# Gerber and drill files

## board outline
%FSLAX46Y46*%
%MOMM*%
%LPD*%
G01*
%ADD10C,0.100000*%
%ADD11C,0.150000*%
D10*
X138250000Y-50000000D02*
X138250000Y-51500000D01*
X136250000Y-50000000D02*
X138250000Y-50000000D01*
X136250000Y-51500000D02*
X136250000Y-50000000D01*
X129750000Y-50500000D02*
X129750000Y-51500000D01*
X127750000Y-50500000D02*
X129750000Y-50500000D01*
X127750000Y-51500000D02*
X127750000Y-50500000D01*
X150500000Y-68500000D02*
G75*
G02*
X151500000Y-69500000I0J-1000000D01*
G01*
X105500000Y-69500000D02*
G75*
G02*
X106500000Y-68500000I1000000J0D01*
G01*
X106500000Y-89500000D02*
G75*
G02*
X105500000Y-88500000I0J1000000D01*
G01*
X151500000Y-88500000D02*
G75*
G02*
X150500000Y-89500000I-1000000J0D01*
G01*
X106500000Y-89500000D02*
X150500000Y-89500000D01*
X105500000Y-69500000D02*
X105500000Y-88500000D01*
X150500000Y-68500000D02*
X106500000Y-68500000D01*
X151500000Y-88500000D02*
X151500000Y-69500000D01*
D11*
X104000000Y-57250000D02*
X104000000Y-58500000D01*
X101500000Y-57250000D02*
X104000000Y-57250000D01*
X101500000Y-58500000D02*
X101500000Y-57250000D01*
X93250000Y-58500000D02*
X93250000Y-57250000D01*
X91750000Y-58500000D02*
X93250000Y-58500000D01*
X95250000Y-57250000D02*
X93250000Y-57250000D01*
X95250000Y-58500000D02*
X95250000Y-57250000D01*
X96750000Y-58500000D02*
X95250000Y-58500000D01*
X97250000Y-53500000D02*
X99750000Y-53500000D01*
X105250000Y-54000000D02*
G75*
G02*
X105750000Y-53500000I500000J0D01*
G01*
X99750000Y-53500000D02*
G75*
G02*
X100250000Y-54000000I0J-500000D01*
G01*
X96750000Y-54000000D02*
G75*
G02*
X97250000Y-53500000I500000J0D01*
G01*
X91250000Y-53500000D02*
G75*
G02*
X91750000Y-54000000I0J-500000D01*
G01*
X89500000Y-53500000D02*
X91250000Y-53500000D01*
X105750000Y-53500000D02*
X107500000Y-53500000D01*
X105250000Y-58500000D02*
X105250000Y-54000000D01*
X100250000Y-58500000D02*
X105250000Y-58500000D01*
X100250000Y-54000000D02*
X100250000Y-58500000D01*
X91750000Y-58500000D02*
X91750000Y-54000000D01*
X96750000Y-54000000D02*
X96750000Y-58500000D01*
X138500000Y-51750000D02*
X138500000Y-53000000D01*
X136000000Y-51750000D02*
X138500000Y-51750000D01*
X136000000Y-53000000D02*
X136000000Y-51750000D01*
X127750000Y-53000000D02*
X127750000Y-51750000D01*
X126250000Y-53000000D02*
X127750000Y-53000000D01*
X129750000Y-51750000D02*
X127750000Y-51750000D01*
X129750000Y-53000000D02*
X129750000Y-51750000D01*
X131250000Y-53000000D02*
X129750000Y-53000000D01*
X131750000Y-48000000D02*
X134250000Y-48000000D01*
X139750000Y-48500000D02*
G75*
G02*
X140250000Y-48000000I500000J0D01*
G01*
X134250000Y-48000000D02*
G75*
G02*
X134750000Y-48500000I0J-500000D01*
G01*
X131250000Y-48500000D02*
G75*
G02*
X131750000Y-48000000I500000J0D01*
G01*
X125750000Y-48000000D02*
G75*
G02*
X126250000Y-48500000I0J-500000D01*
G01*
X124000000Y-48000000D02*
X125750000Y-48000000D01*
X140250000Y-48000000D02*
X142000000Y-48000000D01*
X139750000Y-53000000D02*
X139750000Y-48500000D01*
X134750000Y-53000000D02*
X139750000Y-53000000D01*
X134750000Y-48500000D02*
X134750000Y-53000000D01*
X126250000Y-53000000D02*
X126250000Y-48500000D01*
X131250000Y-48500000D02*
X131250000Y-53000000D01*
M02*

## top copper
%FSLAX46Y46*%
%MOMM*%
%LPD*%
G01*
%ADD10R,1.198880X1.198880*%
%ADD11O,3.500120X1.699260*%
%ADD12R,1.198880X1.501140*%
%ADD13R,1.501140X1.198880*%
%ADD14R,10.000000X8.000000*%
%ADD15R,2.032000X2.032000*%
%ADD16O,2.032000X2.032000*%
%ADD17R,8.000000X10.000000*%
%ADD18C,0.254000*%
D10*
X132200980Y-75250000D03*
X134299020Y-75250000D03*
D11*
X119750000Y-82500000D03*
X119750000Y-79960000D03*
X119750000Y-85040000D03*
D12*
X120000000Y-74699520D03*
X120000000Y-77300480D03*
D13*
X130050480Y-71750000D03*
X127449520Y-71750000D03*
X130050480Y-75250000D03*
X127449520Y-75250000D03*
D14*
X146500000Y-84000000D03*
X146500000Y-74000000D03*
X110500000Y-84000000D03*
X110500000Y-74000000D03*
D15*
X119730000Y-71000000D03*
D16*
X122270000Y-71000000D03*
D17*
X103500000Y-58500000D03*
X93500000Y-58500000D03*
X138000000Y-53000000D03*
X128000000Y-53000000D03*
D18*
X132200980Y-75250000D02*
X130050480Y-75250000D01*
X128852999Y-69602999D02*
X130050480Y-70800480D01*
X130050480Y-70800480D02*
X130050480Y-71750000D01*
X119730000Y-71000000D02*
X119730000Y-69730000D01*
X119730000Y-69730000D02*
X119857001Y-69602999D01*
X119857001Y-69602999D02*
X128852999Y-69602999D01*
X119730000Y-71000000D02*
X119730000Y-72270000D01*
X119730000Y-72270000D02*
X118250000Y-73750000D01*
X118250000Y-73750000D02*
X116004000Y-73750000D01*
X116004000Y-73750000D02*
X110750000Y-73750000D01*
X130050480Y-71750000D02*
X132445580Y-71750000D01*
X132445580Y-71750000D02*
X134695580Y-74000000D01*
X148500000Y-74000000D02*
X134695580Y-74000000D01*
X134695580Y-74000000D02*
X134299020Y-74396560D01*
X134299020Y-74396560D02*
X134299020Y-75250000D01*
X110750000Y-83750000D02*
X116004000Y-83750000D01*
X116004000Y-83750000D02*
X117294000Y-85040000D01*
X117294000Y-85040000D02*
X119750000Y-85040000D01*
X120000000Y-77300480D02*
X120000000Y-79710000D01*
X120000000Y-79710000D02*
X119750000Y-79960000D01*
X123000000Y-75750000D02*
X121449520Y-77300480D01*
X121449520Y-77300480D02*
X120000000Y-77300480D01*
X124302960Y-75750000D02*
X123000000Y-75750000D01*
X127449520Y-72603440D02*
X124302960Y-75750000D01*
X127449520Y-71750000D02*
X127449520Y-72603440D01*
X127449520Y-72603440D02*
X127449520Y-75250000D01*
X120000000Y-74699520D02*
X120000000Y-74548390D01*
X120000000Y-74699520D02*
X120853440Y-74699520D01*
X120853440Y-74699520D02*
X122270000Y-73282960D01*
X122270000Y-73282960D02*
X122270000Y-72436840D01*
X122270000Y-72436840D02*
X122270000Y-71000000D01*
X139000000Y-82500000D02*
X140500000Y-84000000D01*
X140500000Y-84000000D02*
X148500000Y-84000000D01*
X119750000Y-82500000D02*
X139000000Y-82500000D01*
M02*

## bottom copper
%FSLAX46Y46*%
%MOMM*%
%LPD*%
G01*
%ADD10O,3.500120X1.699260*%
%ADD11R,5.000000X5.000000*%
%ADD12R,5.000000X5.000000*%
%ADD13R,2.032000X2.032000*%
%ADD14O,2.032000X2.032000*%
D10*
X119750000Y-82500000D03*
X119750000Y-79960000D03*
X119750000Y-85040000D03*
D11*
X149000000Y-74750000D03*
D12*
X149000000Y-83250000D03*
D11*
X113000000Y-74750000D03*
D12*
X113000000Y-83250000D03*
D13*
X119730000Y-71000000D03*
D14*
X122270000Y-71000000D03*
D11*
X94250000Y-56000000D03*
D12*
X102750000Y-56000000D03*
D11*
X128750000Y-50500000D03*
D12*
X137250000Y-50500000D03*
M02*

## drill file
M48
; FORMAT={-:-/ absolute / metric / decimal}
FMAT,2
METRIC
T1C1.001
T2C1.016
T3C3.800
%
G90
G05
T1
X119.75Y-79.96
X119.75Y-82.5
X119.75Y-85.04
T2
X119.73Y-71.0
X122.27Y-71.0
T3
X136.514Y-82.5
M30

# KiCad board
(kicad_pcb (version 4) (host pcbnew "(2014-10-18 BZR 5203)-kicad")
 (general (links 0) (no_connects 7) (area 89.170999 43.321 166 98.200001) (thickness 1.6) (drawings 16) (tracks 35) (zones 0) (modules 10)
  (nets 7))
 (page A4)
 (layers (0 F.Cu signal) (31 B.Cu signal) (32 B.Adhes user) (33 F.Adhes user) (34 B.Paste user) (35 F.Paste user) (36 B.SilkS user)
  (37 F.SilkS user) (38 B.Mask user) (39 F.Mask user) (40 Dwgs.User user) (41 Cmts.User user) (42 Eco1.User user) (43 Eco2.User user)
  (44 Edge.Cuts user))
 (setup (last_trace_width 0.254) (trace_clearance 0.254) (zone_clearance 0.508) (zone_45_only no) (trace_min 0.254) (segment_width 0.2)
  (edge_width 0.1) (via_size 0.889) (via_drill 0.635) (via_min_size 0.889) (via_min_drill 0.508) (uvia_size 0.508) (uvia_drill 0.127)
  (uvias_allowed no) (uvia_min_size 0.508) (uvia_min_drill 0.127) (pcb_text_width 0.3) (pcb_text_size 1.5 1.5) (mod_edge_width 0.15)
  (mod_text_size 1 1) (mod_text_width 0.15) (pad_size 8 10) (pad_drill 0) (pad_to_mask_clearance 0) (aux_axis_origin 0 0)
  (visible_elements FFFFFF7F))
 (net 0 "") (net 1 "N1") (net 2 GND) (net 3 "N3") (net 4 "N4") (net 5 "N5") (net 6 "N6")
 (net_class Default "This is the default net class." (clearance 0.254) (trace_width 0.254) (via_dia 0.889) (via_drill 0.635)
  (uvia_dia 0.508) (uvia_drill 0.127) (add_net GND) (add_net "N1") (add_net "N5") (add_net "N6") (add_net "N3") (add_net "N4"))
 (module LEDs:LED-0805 (layer F.Cu) (at 133.25 75.25)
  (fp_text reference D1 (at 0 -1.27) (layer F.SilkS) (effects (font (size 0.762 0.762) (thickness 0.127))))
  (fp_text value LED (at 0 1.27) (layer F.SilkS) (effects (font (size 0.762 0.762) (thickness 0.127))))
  (pad 1 smd rect (at -1.04902 0) (size 1.19888 1.19888) (layers F.Cu F.Paste F.Mask) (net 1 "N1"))
  (pad 2 smd rect (at 1.04902 0) (size 1.19888 1.19888) (layers F.Cu F.Paste F.Mask) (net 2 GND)))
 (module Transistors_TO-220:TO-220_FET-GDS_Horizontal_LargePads (layer F.Cu) (at 119.75 82.5 270)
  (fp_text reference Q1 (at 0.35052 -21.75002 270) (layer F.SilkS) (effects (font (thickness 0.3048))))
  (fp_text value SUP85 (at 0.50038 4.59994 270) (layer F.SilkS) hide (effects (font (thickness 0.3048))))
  (pad D thru_hole oval (at 0 0) (size 3.50012 1.69926) (drill 1.00076) (layers *.Cu *.Mask F.SilkS) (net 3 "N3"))
  (pad G thru_hole oval (at -2.54 0) (size 3.50012 1.69926) (drill 1.00076) (layers *.Cu *.Mask F.SilkS) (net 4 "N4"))
  (pad S thru_hole oval (at 2.54 0) (size 3.50012 1.69926) (drill 1.00076) (layers *.Cu *.Mask F.SilkS) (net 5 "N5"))
  (pad "" np_thru_hole circle (at 0 -16.764) (size 3.79984 3.79984) (drill 3.79984) (layers *.Cu *.Mask F.SilkS)))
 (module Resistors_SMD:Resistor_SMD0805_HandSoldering (layer F.Cu) (at 120 76 270)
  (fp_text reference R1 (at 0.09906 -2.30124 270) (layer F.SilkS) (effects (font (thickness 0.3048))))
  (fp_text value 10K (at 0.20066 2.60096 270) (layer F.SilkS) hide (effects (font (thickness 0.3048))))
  (pad 1 smd rect (at -1.30048 0 270) (size 1.50114 1.19888) (layers F.Cu F.Paste F.Mask) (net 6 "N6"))
  (pad 2 smd rect (at 1.30048 0 270) (size 1.50114 1.19888) (layers F.Cu F.Paste F.Mask) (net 4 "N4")))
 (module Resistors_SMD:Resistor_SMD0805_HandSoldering (layer F.Cu) (at 128.75 71.75 180)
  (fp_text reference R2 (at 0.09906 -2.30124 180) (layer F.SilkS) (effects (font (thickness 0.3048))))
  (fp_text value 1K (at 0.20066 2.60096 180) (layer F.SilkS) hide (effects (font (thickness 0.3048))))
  (pad 1 smd rect (at -1.30048 0 180) (size 1.50114 1.19888) (layers F.Cu F.Paste F.Mask) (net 2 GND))
  (pad 2 smd rect (at 1.30048 0 180) (size 1.50114 1.19888) (layers F.Cu F.Paste F.Mask) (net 4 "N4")))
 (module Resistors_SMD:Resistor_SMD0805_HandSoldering (layer F.Cu) (at 128.75 75.25 180)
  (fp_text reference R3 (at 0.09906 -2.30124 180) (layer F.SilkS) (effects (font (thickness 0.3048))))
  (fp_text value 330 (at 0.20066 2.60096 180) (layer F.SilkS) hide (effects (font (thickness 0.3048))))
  (pad 1 smd rect (at -1.30048 0 180) (size 1.50114 1.19888) (layers F.Cu F.Paste F.Mask) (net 1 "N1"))
  (pad 2 smd rect (at 1.30048 0 180) (size 1.50114 1.19888) (layers F.Cu F.Paste F.Mask) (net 4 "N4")))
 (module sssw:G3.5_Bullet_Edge (layer F.Cu) (at 149 79 270)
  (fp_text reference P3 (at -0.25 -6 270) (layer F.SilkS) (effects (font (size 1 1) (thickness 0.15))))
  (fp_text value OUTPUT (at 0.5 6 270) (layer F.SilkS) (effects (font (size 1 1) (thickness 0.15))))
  (pad 1 smd rect (at -4.25 0 270) (size 5 5) (layers B.Cu F.Paste F.Mask) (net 2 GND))
  (pad 2 connect rect (at 4.25 0 270) (size 5 5) (layers B.Cu F.Mask) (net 3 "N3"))
  (pad 2 smd rect (at 5 2.5 270) (size 8 10) (layers F.Cu F.Paste F.Mask) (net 3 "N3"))
  (pad 1 smd rect (at -5 2.5 270) (size 8 10) (layers F.Cu F.Paste F.Mask) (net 2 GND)))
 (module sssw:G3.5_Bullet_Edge (layer F.Cu) (at 113 79 270)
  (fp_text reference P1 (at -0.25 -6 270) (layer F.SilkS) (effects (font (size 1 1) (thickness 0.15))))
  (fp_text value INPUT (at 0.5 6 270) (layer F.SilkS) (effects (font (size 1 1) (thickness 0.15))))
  (pad 1 smd rect (at -4.25 0 270) (size 5 5) (layers B.Cu F.Paste F.Mask) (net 2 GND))
  (pad 2 connect rect (at 4.25 0 270) (size 5 5) (layers B.Cu F.Mask) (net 5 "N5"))
  (pad 2 smd rect (at 5 2.5 270) (size 8 10) (layers F.Cu F.Paste F.Mask) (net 5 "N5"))
  (pad 1 smd rect (at -5 2.5 270) (size 8 10) (layers F.Cu F.Paste F.Mask) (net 2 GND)))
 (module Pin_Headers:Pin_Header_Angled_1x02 (layer F.Cu) (at 121 71)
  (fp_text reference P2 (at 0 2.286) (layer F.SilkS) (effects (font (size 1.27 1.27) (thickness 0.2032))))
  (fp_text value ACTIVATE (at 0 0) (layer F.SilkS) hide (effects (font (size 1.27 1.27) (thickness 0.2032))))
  (pad 1 thru_hole rect (at -1.27 0) (size 2.032 2.032) (drill 1.016) (layers *.Cu *.Mask F.SilkS) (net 2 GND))
  (pad 2 thru_hole oval (at 1.27 0) (size 2.032 2.032) (drill 1.016) (layers *.Cu *.Mask F.SilkS) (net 6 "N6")))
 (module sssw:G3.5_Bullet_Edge (layer F.Cu) (at 98.5 56)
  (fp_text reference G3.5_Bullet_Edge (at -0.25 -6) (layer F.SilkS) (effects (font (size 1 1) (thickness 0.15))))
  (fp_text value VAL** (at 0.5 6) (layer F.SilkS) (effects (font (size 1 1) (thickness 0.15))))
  (fp_line (start 5.5 1.25) (end 5.5 2.5) (layer Edge.Cuts) (width 0.15))
  (fp_line (start 3 1.25) (end 5.5 1.25) (layer Edge.Cuts) (width 0.15))
  (fp_line (start 3 2.5) (end 3 1.25) (layer Edge.Cuts) (width 0.15))
  (fp_line (start -5.25 2.5) (end -5.25 1.25) (layer Edge.Cuts) (width 0.15))
  (fp_line (start -6.75 2.5) (end -5.25 2.5) (layer Edge.Cuts) (width 0.15))
  (fp_line (start -3.25 1.25) (end -5.25 1.25) (layer Edge.Cuts) (width 0.15))
  (fp_line (start -3.25 2.5) (end -3.25 1.25) (layer Edge.Cuts) (width 0.15))
  (fp_line (start -1.75 2.5) (end -3.25 2.5) (layer Edge.Cuts) (width 0.15))
  (fp_line (start -1.25 -2.5) (end 1.25 -2.5) (layer Edge.Cuts) (width 0.15))
  (fp_arc (start 7.25 -2) (end 6.75 -2) (angle 90) (layer Edge.Cuts) (width 0.15))
  (fp_arc (start 1.25 -2) (end 1.25 -2.5) (angle 90) (layer Edge.Cuts) (width 0.15))
  (fp_arc (start -1.25 -2) (end -1.75 -2) (angle 90) (layer Edge.Cuts) (width 0.15))
  (fp_arc (start -7.25 -2) (end -7.25 -2.5) (angle 90) (layer Edge.Cuts) (width 0.15))
  (fp_line (start -9 -2.5) (end -7.25 -2.5) (layer Edge.Cuts) (width 0.15))
  (fp_line (start 7.25 -2.5) (end 9 -2.5) (layer Edge.Cuts) (width 0.15))
  (fp_line (start 6.75 2.5) (end 6.75 -2) (layer Edge.Cuts) (width 0.15))
  (fp_line (start 1.75 2.5) (end 6.75 2.5) (layer Edge.Cuts) (width 0.15))
  (fp_line (start 1.75 -2) (end 1.75 2.5) (layer Edge.Cuts) (width 0.15))
  (fp_line (start -6.75 2.5) (end -6.75 -2) (layer Edge.Cuts) (width 0.15))
  (fp_line (start -1.75 -2) (end -1.75 2.5) (layer Edge.Cuts) (width 0.15))
  (pad 1 smd rect (at -4.25 0) (size 5 5) (layers B.Cu F.Paste F.Mask))
  (pad 2 connect rect (at 4.25 0) (size 5 5) (layers B.Cu F.Mask))
  (pad 2 smd rect (at 5 2.5) (size 8 10) (layers F.Cu F.Paste F.Mask))
  (pad 1 smd rect (at -5 2.5) (size 8 10) (layers F.Cu F.Paste F.Mask)))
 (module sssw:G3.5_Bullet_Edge (layer F.Cu) (at 133 50.5)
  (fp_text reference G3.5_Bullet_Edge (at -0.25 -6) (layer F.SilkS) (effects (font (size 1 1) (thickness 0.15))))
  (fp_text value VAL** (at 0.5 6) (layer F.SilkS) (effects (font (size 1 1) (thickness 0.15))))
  (fp_line (start 5.5 1.25) (end 5.5 2.5) (layer Edge.Cuts) (width 0.15))
  (fp_line (start 3 1.25) (end 5.5 1.25) (layer Edge.Cuts) (width 0.15))
  (fp_line (start 3 2.5) (end 3 1.25) (layer Edge.Cuts) (width 0.15))
  (fp_line (start -5.25 2.5) (end -5.25 1.25) (layer Edge.Cuts) (width 0.15))
  (fp_line (start -6.75 2.5) (end -5.25 2.5) (layer Edge.Cuts) (width 0.15))
  (fp_line (start -3.25 1.25) (end -5.25 1.25) (layer Edge.Cuts) (width 0.15))
  (fp_line (start -3.25 2.5) (end -3.25 1.25) (layer Edge.Cuts) (width 0.15))
  (fp_line (start -1.75 2.5) (end -3.25 2.5) (layer Edge.Cuts) (width 0.15))
  (fp_line (start -1.25 -2.5) (end 1.25 -2.5) (layer Edge.Cuts) (width 0.15))
  (fp_arc (start 7.25 -2) (end 6.75 -2) (angle 90) (layer Edge.Cuts) (width 0.15))
  (fp_arc (start 1.25 -2) (end 1.25 -2.5) (angle 90) (layer Edge.Cuts) (width 0.15))
  (fp_arc (start -1.25 -2) (end -1.75 -2) (angle 90) (layer Edge.Cuts) (width 0.15))
  (fp_arc (start -7.25 -2) (end -7.25 -2.5) (angle 90) (layer Edge.Cuts) (width 0.15))
  (fp_line (start -9 -2.5) (end -7.25 -2.5) (layer Edge.Cuts) (width 0.15))
  (fp_line (start 7.25 -2.5) (end 9 -2.5) (layer Edge.Cuts) (width 0.15))
  (fp_line (start 6.75 2.5) (end 6.75 -2) (layer Edge.Cuts) (width 0.15))
  (fp_line (start 1.75 2.5) (end 6.75 2.5) (layer Edge.Cuts) (width 0.15))
  (fp_line (start 1.75 -2) (end 1.75 2.5) (layer Edge.Cuts) (width 0.15))
  (fp_line (start -6.75 2.5) (end -6.75 -2) (layer Edge.Cuts) (width 0.15))
  (fp_line (start -1.75 -2) (end -1.75 2.5) (layer Edge.Cuts) (width 0.15))
  (pad 1 smd rect (at -4.25 0) (size 5 5) (layers B.Cu F.Paste F.Mask))
  (pad 2 connect rect (at 4.25 0) (size 5 5) (layers B.Cu F.Mask))
  (pad 2 smd rect (at 5 2.5) (size 8 10) (layers F.Cu F.Paste F.Mask))
  (pad 1 smd rect (at -5 2.5) (size 8 10) (layers F.Cu F.Paste F.Mask)))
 (gr_line (start 138.25 50) (end 138.25 51.5) (layer Edge.Cuts) (width 0.1))
 (gr_line (start 136.25 50) (end 138.25 50) (layer Edge.Cuts) (width 0.1))
 (gr_line (start 136.25 51.5) (end 136.25 50) (layer Edge.Cuts) (width 0.1))
 (gr_line (start 129.75 50.5) (end 129.75 51.5) (layer Edge.Cuts) (width 0.1))
 (gr_line (start 127.75 50.5) (end 129.75 50.5) (layer Edge.Cuts) (width 0.1))
 (gr_line (start 127.75 51.5) (end 127.75 50.5) (layer Edge.Cuts) (width 0.1))
 (gr_arc (start 150.5 69.5) (end 151.5 69.5) (angle -90) (layer Edge.Cuts) (width 0.1))
 (gr_arc (start 106.5 69.5) (end 106.5 68.5) (angle -90) (layer Edge.Cuts) (width 0.1))
 (gr_arc (start 106.5 88.5) (end 105.5 88.5) (angle -90) (layer Edge.Cuts) (width 0.1))
 (gr_arc (start 150.5 88.5) (end 151.5 88.5) (angle 90) (layer Edge.Cuts) (width 0.1))
 (gr_line (start 106.5 89.5) (end 150.5 89.5) (layer Edge.Cuts) (width 0.1))
 (gr_line (start 105.5 69.5) (end 105.5 88.5) (layer Edge.Cuts) (width 0.1))
 (gr_line (start 150.5 68.5) (end 106.5 68.5) (layer Edge.Cuts) (width 0.1))
 (gr_line (start 151.5 88.5) (end 151.5 69.5) (layer Edge.Cuts) (width 0.1))
 (segment (start 132.20098 75.25) (end 130.05048 75.25) (width 0.254) (layer F.Cu) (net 1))
 (segment (start 128.852999 69.602999) (end 130.05048 70.80048) (width 0.254) (layer F.Cu) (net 2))
 (segment (start 130.05048 70.80048) (end 130.05048 71.75) (width 0.254) (layer F.Cu) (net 2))
 (segment (start 119.73 71) (end 119.73 69.73) (width 0.254) (layer F.Cu) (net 2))
 (segment (start 119.73 69.73) (end 119.857001 69.602999) (width 0.254) (layer F.Cu) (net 2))
 (segment (start 119.857001 69.602999) (end 128.852999 69.602999) (width 0.254) (layer F.Cu) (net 2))
 (segment (start 119.73 71) (end 119.73 72.27) (width 0.254) (layer F.Cu) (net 2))
 (segment (start 119.73 72.27) (end 118.25 73.75) (width 0.254) (layer F.Cu) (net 2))
 (segment (start 118.25 73.75) (end 116.004 73.75) (width 0.254) (layer F.Cu) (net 2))
 (segment (start 116.004 73.75) (end 110.75 73.75) (width 0.254) (layer F.Cu) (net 2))
 (segment (start 130.05048 71.75) (end 132.44558 71.75) (width 0.254) (layer F.Cu) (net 2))
 (segment (start 132.44558 71.75) (end 134.69558 74) (width 0.254) (layer F.Cu) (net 2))
 (segment (start 148.5 74) (end 134.69558 74) (width 0.254) (layer F.Cu) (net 2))
 (segment (start 134.69558 74) (end 134.29902 74.39656) (width 0.254) (layer F.Cu) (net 2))
 (segment (start 134.29902 74.39656) (end 134.29902 75.25) (width 0.254) (layer F.Cu) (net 2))
 (segment (start 110.75 83.75) (end 116.004 83.75) (width 0.254) (layer F.Cu) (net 5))
 (segment (start 116.004 83.75) (end 117.294 85.04) (width 0.254) (layer F.Cu) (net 5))
 (segment (start 117.294 85.04) (end 119.75 85.04) (width 0.254) (layer F.Cu) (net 5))
 (segment (start 120 77.30048) (end 120 79.71) (width 0.254) (layer F.Cu) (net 4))
 (segment (start 120 79.71) (end 119.75 79.96) (width 0.254) (layer F.Cu) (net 4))
 (segment (start 119.75 79.96) (end 119.75 80) (width 0.254) (layer Edge.Cuts) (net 4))
 (segment (start 123 75.75) (end 121.44952 77.30048) (width 0.254) (layer F.Cu) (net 4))
 (segment (start 121.44952 77.30048) (end 120 77.30048) (width 0.254) (layer F.Cu) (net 4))
 (segment (start 124.30296 75.75) (end 123 75.75) (width 0.254) (layer F.Cu) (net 4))
 (segment (start 127.44952 72.60344) (end 124.30296 75.75) (width 0.254) (layer F.Cu) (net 4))
 (segment (start 127.44952 71.75) (end 127.44952 72.60344) (width 0.254) (layer F.Cu) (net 4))
 (segment (start 127.44952 72.60344) (end 127.44952 75.25) (width 0.254) (layer F.Cu) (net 4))
 (segment (start 120 74.69952) (end 120 74.54839) (width 0.254) (layer F.Cu) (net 6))
 (segment (start 120 74.69952) (end 120.85344 74.69952) (width 0.254) (layer F.Cu) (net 6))
 (segment (start 120.85344 74.69952) (end 122.27 73.28296) (width 0.254) (layer F.Cu) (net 6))
 (segment (start 122.27 73.28296) (end 122.27 72.43684) (width 0.254) (layer F.Cu) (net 6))
 (segment (start 122.27 72.43684) (end 122.27 71) (width 0.254) (layer F.Cu) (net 6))
 (segment (start 139 82.5) (end 140.5 84) (width 0.254) (layer F.Cu) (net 3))
 (segment (start 140.5 84) (end 148.5 84) (width 0.254) (layer F.Cu) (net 3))
 (segment (start 119.75 82.5) (end 139 82.5) (width 0.254) (layer F.Cu) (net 3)))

